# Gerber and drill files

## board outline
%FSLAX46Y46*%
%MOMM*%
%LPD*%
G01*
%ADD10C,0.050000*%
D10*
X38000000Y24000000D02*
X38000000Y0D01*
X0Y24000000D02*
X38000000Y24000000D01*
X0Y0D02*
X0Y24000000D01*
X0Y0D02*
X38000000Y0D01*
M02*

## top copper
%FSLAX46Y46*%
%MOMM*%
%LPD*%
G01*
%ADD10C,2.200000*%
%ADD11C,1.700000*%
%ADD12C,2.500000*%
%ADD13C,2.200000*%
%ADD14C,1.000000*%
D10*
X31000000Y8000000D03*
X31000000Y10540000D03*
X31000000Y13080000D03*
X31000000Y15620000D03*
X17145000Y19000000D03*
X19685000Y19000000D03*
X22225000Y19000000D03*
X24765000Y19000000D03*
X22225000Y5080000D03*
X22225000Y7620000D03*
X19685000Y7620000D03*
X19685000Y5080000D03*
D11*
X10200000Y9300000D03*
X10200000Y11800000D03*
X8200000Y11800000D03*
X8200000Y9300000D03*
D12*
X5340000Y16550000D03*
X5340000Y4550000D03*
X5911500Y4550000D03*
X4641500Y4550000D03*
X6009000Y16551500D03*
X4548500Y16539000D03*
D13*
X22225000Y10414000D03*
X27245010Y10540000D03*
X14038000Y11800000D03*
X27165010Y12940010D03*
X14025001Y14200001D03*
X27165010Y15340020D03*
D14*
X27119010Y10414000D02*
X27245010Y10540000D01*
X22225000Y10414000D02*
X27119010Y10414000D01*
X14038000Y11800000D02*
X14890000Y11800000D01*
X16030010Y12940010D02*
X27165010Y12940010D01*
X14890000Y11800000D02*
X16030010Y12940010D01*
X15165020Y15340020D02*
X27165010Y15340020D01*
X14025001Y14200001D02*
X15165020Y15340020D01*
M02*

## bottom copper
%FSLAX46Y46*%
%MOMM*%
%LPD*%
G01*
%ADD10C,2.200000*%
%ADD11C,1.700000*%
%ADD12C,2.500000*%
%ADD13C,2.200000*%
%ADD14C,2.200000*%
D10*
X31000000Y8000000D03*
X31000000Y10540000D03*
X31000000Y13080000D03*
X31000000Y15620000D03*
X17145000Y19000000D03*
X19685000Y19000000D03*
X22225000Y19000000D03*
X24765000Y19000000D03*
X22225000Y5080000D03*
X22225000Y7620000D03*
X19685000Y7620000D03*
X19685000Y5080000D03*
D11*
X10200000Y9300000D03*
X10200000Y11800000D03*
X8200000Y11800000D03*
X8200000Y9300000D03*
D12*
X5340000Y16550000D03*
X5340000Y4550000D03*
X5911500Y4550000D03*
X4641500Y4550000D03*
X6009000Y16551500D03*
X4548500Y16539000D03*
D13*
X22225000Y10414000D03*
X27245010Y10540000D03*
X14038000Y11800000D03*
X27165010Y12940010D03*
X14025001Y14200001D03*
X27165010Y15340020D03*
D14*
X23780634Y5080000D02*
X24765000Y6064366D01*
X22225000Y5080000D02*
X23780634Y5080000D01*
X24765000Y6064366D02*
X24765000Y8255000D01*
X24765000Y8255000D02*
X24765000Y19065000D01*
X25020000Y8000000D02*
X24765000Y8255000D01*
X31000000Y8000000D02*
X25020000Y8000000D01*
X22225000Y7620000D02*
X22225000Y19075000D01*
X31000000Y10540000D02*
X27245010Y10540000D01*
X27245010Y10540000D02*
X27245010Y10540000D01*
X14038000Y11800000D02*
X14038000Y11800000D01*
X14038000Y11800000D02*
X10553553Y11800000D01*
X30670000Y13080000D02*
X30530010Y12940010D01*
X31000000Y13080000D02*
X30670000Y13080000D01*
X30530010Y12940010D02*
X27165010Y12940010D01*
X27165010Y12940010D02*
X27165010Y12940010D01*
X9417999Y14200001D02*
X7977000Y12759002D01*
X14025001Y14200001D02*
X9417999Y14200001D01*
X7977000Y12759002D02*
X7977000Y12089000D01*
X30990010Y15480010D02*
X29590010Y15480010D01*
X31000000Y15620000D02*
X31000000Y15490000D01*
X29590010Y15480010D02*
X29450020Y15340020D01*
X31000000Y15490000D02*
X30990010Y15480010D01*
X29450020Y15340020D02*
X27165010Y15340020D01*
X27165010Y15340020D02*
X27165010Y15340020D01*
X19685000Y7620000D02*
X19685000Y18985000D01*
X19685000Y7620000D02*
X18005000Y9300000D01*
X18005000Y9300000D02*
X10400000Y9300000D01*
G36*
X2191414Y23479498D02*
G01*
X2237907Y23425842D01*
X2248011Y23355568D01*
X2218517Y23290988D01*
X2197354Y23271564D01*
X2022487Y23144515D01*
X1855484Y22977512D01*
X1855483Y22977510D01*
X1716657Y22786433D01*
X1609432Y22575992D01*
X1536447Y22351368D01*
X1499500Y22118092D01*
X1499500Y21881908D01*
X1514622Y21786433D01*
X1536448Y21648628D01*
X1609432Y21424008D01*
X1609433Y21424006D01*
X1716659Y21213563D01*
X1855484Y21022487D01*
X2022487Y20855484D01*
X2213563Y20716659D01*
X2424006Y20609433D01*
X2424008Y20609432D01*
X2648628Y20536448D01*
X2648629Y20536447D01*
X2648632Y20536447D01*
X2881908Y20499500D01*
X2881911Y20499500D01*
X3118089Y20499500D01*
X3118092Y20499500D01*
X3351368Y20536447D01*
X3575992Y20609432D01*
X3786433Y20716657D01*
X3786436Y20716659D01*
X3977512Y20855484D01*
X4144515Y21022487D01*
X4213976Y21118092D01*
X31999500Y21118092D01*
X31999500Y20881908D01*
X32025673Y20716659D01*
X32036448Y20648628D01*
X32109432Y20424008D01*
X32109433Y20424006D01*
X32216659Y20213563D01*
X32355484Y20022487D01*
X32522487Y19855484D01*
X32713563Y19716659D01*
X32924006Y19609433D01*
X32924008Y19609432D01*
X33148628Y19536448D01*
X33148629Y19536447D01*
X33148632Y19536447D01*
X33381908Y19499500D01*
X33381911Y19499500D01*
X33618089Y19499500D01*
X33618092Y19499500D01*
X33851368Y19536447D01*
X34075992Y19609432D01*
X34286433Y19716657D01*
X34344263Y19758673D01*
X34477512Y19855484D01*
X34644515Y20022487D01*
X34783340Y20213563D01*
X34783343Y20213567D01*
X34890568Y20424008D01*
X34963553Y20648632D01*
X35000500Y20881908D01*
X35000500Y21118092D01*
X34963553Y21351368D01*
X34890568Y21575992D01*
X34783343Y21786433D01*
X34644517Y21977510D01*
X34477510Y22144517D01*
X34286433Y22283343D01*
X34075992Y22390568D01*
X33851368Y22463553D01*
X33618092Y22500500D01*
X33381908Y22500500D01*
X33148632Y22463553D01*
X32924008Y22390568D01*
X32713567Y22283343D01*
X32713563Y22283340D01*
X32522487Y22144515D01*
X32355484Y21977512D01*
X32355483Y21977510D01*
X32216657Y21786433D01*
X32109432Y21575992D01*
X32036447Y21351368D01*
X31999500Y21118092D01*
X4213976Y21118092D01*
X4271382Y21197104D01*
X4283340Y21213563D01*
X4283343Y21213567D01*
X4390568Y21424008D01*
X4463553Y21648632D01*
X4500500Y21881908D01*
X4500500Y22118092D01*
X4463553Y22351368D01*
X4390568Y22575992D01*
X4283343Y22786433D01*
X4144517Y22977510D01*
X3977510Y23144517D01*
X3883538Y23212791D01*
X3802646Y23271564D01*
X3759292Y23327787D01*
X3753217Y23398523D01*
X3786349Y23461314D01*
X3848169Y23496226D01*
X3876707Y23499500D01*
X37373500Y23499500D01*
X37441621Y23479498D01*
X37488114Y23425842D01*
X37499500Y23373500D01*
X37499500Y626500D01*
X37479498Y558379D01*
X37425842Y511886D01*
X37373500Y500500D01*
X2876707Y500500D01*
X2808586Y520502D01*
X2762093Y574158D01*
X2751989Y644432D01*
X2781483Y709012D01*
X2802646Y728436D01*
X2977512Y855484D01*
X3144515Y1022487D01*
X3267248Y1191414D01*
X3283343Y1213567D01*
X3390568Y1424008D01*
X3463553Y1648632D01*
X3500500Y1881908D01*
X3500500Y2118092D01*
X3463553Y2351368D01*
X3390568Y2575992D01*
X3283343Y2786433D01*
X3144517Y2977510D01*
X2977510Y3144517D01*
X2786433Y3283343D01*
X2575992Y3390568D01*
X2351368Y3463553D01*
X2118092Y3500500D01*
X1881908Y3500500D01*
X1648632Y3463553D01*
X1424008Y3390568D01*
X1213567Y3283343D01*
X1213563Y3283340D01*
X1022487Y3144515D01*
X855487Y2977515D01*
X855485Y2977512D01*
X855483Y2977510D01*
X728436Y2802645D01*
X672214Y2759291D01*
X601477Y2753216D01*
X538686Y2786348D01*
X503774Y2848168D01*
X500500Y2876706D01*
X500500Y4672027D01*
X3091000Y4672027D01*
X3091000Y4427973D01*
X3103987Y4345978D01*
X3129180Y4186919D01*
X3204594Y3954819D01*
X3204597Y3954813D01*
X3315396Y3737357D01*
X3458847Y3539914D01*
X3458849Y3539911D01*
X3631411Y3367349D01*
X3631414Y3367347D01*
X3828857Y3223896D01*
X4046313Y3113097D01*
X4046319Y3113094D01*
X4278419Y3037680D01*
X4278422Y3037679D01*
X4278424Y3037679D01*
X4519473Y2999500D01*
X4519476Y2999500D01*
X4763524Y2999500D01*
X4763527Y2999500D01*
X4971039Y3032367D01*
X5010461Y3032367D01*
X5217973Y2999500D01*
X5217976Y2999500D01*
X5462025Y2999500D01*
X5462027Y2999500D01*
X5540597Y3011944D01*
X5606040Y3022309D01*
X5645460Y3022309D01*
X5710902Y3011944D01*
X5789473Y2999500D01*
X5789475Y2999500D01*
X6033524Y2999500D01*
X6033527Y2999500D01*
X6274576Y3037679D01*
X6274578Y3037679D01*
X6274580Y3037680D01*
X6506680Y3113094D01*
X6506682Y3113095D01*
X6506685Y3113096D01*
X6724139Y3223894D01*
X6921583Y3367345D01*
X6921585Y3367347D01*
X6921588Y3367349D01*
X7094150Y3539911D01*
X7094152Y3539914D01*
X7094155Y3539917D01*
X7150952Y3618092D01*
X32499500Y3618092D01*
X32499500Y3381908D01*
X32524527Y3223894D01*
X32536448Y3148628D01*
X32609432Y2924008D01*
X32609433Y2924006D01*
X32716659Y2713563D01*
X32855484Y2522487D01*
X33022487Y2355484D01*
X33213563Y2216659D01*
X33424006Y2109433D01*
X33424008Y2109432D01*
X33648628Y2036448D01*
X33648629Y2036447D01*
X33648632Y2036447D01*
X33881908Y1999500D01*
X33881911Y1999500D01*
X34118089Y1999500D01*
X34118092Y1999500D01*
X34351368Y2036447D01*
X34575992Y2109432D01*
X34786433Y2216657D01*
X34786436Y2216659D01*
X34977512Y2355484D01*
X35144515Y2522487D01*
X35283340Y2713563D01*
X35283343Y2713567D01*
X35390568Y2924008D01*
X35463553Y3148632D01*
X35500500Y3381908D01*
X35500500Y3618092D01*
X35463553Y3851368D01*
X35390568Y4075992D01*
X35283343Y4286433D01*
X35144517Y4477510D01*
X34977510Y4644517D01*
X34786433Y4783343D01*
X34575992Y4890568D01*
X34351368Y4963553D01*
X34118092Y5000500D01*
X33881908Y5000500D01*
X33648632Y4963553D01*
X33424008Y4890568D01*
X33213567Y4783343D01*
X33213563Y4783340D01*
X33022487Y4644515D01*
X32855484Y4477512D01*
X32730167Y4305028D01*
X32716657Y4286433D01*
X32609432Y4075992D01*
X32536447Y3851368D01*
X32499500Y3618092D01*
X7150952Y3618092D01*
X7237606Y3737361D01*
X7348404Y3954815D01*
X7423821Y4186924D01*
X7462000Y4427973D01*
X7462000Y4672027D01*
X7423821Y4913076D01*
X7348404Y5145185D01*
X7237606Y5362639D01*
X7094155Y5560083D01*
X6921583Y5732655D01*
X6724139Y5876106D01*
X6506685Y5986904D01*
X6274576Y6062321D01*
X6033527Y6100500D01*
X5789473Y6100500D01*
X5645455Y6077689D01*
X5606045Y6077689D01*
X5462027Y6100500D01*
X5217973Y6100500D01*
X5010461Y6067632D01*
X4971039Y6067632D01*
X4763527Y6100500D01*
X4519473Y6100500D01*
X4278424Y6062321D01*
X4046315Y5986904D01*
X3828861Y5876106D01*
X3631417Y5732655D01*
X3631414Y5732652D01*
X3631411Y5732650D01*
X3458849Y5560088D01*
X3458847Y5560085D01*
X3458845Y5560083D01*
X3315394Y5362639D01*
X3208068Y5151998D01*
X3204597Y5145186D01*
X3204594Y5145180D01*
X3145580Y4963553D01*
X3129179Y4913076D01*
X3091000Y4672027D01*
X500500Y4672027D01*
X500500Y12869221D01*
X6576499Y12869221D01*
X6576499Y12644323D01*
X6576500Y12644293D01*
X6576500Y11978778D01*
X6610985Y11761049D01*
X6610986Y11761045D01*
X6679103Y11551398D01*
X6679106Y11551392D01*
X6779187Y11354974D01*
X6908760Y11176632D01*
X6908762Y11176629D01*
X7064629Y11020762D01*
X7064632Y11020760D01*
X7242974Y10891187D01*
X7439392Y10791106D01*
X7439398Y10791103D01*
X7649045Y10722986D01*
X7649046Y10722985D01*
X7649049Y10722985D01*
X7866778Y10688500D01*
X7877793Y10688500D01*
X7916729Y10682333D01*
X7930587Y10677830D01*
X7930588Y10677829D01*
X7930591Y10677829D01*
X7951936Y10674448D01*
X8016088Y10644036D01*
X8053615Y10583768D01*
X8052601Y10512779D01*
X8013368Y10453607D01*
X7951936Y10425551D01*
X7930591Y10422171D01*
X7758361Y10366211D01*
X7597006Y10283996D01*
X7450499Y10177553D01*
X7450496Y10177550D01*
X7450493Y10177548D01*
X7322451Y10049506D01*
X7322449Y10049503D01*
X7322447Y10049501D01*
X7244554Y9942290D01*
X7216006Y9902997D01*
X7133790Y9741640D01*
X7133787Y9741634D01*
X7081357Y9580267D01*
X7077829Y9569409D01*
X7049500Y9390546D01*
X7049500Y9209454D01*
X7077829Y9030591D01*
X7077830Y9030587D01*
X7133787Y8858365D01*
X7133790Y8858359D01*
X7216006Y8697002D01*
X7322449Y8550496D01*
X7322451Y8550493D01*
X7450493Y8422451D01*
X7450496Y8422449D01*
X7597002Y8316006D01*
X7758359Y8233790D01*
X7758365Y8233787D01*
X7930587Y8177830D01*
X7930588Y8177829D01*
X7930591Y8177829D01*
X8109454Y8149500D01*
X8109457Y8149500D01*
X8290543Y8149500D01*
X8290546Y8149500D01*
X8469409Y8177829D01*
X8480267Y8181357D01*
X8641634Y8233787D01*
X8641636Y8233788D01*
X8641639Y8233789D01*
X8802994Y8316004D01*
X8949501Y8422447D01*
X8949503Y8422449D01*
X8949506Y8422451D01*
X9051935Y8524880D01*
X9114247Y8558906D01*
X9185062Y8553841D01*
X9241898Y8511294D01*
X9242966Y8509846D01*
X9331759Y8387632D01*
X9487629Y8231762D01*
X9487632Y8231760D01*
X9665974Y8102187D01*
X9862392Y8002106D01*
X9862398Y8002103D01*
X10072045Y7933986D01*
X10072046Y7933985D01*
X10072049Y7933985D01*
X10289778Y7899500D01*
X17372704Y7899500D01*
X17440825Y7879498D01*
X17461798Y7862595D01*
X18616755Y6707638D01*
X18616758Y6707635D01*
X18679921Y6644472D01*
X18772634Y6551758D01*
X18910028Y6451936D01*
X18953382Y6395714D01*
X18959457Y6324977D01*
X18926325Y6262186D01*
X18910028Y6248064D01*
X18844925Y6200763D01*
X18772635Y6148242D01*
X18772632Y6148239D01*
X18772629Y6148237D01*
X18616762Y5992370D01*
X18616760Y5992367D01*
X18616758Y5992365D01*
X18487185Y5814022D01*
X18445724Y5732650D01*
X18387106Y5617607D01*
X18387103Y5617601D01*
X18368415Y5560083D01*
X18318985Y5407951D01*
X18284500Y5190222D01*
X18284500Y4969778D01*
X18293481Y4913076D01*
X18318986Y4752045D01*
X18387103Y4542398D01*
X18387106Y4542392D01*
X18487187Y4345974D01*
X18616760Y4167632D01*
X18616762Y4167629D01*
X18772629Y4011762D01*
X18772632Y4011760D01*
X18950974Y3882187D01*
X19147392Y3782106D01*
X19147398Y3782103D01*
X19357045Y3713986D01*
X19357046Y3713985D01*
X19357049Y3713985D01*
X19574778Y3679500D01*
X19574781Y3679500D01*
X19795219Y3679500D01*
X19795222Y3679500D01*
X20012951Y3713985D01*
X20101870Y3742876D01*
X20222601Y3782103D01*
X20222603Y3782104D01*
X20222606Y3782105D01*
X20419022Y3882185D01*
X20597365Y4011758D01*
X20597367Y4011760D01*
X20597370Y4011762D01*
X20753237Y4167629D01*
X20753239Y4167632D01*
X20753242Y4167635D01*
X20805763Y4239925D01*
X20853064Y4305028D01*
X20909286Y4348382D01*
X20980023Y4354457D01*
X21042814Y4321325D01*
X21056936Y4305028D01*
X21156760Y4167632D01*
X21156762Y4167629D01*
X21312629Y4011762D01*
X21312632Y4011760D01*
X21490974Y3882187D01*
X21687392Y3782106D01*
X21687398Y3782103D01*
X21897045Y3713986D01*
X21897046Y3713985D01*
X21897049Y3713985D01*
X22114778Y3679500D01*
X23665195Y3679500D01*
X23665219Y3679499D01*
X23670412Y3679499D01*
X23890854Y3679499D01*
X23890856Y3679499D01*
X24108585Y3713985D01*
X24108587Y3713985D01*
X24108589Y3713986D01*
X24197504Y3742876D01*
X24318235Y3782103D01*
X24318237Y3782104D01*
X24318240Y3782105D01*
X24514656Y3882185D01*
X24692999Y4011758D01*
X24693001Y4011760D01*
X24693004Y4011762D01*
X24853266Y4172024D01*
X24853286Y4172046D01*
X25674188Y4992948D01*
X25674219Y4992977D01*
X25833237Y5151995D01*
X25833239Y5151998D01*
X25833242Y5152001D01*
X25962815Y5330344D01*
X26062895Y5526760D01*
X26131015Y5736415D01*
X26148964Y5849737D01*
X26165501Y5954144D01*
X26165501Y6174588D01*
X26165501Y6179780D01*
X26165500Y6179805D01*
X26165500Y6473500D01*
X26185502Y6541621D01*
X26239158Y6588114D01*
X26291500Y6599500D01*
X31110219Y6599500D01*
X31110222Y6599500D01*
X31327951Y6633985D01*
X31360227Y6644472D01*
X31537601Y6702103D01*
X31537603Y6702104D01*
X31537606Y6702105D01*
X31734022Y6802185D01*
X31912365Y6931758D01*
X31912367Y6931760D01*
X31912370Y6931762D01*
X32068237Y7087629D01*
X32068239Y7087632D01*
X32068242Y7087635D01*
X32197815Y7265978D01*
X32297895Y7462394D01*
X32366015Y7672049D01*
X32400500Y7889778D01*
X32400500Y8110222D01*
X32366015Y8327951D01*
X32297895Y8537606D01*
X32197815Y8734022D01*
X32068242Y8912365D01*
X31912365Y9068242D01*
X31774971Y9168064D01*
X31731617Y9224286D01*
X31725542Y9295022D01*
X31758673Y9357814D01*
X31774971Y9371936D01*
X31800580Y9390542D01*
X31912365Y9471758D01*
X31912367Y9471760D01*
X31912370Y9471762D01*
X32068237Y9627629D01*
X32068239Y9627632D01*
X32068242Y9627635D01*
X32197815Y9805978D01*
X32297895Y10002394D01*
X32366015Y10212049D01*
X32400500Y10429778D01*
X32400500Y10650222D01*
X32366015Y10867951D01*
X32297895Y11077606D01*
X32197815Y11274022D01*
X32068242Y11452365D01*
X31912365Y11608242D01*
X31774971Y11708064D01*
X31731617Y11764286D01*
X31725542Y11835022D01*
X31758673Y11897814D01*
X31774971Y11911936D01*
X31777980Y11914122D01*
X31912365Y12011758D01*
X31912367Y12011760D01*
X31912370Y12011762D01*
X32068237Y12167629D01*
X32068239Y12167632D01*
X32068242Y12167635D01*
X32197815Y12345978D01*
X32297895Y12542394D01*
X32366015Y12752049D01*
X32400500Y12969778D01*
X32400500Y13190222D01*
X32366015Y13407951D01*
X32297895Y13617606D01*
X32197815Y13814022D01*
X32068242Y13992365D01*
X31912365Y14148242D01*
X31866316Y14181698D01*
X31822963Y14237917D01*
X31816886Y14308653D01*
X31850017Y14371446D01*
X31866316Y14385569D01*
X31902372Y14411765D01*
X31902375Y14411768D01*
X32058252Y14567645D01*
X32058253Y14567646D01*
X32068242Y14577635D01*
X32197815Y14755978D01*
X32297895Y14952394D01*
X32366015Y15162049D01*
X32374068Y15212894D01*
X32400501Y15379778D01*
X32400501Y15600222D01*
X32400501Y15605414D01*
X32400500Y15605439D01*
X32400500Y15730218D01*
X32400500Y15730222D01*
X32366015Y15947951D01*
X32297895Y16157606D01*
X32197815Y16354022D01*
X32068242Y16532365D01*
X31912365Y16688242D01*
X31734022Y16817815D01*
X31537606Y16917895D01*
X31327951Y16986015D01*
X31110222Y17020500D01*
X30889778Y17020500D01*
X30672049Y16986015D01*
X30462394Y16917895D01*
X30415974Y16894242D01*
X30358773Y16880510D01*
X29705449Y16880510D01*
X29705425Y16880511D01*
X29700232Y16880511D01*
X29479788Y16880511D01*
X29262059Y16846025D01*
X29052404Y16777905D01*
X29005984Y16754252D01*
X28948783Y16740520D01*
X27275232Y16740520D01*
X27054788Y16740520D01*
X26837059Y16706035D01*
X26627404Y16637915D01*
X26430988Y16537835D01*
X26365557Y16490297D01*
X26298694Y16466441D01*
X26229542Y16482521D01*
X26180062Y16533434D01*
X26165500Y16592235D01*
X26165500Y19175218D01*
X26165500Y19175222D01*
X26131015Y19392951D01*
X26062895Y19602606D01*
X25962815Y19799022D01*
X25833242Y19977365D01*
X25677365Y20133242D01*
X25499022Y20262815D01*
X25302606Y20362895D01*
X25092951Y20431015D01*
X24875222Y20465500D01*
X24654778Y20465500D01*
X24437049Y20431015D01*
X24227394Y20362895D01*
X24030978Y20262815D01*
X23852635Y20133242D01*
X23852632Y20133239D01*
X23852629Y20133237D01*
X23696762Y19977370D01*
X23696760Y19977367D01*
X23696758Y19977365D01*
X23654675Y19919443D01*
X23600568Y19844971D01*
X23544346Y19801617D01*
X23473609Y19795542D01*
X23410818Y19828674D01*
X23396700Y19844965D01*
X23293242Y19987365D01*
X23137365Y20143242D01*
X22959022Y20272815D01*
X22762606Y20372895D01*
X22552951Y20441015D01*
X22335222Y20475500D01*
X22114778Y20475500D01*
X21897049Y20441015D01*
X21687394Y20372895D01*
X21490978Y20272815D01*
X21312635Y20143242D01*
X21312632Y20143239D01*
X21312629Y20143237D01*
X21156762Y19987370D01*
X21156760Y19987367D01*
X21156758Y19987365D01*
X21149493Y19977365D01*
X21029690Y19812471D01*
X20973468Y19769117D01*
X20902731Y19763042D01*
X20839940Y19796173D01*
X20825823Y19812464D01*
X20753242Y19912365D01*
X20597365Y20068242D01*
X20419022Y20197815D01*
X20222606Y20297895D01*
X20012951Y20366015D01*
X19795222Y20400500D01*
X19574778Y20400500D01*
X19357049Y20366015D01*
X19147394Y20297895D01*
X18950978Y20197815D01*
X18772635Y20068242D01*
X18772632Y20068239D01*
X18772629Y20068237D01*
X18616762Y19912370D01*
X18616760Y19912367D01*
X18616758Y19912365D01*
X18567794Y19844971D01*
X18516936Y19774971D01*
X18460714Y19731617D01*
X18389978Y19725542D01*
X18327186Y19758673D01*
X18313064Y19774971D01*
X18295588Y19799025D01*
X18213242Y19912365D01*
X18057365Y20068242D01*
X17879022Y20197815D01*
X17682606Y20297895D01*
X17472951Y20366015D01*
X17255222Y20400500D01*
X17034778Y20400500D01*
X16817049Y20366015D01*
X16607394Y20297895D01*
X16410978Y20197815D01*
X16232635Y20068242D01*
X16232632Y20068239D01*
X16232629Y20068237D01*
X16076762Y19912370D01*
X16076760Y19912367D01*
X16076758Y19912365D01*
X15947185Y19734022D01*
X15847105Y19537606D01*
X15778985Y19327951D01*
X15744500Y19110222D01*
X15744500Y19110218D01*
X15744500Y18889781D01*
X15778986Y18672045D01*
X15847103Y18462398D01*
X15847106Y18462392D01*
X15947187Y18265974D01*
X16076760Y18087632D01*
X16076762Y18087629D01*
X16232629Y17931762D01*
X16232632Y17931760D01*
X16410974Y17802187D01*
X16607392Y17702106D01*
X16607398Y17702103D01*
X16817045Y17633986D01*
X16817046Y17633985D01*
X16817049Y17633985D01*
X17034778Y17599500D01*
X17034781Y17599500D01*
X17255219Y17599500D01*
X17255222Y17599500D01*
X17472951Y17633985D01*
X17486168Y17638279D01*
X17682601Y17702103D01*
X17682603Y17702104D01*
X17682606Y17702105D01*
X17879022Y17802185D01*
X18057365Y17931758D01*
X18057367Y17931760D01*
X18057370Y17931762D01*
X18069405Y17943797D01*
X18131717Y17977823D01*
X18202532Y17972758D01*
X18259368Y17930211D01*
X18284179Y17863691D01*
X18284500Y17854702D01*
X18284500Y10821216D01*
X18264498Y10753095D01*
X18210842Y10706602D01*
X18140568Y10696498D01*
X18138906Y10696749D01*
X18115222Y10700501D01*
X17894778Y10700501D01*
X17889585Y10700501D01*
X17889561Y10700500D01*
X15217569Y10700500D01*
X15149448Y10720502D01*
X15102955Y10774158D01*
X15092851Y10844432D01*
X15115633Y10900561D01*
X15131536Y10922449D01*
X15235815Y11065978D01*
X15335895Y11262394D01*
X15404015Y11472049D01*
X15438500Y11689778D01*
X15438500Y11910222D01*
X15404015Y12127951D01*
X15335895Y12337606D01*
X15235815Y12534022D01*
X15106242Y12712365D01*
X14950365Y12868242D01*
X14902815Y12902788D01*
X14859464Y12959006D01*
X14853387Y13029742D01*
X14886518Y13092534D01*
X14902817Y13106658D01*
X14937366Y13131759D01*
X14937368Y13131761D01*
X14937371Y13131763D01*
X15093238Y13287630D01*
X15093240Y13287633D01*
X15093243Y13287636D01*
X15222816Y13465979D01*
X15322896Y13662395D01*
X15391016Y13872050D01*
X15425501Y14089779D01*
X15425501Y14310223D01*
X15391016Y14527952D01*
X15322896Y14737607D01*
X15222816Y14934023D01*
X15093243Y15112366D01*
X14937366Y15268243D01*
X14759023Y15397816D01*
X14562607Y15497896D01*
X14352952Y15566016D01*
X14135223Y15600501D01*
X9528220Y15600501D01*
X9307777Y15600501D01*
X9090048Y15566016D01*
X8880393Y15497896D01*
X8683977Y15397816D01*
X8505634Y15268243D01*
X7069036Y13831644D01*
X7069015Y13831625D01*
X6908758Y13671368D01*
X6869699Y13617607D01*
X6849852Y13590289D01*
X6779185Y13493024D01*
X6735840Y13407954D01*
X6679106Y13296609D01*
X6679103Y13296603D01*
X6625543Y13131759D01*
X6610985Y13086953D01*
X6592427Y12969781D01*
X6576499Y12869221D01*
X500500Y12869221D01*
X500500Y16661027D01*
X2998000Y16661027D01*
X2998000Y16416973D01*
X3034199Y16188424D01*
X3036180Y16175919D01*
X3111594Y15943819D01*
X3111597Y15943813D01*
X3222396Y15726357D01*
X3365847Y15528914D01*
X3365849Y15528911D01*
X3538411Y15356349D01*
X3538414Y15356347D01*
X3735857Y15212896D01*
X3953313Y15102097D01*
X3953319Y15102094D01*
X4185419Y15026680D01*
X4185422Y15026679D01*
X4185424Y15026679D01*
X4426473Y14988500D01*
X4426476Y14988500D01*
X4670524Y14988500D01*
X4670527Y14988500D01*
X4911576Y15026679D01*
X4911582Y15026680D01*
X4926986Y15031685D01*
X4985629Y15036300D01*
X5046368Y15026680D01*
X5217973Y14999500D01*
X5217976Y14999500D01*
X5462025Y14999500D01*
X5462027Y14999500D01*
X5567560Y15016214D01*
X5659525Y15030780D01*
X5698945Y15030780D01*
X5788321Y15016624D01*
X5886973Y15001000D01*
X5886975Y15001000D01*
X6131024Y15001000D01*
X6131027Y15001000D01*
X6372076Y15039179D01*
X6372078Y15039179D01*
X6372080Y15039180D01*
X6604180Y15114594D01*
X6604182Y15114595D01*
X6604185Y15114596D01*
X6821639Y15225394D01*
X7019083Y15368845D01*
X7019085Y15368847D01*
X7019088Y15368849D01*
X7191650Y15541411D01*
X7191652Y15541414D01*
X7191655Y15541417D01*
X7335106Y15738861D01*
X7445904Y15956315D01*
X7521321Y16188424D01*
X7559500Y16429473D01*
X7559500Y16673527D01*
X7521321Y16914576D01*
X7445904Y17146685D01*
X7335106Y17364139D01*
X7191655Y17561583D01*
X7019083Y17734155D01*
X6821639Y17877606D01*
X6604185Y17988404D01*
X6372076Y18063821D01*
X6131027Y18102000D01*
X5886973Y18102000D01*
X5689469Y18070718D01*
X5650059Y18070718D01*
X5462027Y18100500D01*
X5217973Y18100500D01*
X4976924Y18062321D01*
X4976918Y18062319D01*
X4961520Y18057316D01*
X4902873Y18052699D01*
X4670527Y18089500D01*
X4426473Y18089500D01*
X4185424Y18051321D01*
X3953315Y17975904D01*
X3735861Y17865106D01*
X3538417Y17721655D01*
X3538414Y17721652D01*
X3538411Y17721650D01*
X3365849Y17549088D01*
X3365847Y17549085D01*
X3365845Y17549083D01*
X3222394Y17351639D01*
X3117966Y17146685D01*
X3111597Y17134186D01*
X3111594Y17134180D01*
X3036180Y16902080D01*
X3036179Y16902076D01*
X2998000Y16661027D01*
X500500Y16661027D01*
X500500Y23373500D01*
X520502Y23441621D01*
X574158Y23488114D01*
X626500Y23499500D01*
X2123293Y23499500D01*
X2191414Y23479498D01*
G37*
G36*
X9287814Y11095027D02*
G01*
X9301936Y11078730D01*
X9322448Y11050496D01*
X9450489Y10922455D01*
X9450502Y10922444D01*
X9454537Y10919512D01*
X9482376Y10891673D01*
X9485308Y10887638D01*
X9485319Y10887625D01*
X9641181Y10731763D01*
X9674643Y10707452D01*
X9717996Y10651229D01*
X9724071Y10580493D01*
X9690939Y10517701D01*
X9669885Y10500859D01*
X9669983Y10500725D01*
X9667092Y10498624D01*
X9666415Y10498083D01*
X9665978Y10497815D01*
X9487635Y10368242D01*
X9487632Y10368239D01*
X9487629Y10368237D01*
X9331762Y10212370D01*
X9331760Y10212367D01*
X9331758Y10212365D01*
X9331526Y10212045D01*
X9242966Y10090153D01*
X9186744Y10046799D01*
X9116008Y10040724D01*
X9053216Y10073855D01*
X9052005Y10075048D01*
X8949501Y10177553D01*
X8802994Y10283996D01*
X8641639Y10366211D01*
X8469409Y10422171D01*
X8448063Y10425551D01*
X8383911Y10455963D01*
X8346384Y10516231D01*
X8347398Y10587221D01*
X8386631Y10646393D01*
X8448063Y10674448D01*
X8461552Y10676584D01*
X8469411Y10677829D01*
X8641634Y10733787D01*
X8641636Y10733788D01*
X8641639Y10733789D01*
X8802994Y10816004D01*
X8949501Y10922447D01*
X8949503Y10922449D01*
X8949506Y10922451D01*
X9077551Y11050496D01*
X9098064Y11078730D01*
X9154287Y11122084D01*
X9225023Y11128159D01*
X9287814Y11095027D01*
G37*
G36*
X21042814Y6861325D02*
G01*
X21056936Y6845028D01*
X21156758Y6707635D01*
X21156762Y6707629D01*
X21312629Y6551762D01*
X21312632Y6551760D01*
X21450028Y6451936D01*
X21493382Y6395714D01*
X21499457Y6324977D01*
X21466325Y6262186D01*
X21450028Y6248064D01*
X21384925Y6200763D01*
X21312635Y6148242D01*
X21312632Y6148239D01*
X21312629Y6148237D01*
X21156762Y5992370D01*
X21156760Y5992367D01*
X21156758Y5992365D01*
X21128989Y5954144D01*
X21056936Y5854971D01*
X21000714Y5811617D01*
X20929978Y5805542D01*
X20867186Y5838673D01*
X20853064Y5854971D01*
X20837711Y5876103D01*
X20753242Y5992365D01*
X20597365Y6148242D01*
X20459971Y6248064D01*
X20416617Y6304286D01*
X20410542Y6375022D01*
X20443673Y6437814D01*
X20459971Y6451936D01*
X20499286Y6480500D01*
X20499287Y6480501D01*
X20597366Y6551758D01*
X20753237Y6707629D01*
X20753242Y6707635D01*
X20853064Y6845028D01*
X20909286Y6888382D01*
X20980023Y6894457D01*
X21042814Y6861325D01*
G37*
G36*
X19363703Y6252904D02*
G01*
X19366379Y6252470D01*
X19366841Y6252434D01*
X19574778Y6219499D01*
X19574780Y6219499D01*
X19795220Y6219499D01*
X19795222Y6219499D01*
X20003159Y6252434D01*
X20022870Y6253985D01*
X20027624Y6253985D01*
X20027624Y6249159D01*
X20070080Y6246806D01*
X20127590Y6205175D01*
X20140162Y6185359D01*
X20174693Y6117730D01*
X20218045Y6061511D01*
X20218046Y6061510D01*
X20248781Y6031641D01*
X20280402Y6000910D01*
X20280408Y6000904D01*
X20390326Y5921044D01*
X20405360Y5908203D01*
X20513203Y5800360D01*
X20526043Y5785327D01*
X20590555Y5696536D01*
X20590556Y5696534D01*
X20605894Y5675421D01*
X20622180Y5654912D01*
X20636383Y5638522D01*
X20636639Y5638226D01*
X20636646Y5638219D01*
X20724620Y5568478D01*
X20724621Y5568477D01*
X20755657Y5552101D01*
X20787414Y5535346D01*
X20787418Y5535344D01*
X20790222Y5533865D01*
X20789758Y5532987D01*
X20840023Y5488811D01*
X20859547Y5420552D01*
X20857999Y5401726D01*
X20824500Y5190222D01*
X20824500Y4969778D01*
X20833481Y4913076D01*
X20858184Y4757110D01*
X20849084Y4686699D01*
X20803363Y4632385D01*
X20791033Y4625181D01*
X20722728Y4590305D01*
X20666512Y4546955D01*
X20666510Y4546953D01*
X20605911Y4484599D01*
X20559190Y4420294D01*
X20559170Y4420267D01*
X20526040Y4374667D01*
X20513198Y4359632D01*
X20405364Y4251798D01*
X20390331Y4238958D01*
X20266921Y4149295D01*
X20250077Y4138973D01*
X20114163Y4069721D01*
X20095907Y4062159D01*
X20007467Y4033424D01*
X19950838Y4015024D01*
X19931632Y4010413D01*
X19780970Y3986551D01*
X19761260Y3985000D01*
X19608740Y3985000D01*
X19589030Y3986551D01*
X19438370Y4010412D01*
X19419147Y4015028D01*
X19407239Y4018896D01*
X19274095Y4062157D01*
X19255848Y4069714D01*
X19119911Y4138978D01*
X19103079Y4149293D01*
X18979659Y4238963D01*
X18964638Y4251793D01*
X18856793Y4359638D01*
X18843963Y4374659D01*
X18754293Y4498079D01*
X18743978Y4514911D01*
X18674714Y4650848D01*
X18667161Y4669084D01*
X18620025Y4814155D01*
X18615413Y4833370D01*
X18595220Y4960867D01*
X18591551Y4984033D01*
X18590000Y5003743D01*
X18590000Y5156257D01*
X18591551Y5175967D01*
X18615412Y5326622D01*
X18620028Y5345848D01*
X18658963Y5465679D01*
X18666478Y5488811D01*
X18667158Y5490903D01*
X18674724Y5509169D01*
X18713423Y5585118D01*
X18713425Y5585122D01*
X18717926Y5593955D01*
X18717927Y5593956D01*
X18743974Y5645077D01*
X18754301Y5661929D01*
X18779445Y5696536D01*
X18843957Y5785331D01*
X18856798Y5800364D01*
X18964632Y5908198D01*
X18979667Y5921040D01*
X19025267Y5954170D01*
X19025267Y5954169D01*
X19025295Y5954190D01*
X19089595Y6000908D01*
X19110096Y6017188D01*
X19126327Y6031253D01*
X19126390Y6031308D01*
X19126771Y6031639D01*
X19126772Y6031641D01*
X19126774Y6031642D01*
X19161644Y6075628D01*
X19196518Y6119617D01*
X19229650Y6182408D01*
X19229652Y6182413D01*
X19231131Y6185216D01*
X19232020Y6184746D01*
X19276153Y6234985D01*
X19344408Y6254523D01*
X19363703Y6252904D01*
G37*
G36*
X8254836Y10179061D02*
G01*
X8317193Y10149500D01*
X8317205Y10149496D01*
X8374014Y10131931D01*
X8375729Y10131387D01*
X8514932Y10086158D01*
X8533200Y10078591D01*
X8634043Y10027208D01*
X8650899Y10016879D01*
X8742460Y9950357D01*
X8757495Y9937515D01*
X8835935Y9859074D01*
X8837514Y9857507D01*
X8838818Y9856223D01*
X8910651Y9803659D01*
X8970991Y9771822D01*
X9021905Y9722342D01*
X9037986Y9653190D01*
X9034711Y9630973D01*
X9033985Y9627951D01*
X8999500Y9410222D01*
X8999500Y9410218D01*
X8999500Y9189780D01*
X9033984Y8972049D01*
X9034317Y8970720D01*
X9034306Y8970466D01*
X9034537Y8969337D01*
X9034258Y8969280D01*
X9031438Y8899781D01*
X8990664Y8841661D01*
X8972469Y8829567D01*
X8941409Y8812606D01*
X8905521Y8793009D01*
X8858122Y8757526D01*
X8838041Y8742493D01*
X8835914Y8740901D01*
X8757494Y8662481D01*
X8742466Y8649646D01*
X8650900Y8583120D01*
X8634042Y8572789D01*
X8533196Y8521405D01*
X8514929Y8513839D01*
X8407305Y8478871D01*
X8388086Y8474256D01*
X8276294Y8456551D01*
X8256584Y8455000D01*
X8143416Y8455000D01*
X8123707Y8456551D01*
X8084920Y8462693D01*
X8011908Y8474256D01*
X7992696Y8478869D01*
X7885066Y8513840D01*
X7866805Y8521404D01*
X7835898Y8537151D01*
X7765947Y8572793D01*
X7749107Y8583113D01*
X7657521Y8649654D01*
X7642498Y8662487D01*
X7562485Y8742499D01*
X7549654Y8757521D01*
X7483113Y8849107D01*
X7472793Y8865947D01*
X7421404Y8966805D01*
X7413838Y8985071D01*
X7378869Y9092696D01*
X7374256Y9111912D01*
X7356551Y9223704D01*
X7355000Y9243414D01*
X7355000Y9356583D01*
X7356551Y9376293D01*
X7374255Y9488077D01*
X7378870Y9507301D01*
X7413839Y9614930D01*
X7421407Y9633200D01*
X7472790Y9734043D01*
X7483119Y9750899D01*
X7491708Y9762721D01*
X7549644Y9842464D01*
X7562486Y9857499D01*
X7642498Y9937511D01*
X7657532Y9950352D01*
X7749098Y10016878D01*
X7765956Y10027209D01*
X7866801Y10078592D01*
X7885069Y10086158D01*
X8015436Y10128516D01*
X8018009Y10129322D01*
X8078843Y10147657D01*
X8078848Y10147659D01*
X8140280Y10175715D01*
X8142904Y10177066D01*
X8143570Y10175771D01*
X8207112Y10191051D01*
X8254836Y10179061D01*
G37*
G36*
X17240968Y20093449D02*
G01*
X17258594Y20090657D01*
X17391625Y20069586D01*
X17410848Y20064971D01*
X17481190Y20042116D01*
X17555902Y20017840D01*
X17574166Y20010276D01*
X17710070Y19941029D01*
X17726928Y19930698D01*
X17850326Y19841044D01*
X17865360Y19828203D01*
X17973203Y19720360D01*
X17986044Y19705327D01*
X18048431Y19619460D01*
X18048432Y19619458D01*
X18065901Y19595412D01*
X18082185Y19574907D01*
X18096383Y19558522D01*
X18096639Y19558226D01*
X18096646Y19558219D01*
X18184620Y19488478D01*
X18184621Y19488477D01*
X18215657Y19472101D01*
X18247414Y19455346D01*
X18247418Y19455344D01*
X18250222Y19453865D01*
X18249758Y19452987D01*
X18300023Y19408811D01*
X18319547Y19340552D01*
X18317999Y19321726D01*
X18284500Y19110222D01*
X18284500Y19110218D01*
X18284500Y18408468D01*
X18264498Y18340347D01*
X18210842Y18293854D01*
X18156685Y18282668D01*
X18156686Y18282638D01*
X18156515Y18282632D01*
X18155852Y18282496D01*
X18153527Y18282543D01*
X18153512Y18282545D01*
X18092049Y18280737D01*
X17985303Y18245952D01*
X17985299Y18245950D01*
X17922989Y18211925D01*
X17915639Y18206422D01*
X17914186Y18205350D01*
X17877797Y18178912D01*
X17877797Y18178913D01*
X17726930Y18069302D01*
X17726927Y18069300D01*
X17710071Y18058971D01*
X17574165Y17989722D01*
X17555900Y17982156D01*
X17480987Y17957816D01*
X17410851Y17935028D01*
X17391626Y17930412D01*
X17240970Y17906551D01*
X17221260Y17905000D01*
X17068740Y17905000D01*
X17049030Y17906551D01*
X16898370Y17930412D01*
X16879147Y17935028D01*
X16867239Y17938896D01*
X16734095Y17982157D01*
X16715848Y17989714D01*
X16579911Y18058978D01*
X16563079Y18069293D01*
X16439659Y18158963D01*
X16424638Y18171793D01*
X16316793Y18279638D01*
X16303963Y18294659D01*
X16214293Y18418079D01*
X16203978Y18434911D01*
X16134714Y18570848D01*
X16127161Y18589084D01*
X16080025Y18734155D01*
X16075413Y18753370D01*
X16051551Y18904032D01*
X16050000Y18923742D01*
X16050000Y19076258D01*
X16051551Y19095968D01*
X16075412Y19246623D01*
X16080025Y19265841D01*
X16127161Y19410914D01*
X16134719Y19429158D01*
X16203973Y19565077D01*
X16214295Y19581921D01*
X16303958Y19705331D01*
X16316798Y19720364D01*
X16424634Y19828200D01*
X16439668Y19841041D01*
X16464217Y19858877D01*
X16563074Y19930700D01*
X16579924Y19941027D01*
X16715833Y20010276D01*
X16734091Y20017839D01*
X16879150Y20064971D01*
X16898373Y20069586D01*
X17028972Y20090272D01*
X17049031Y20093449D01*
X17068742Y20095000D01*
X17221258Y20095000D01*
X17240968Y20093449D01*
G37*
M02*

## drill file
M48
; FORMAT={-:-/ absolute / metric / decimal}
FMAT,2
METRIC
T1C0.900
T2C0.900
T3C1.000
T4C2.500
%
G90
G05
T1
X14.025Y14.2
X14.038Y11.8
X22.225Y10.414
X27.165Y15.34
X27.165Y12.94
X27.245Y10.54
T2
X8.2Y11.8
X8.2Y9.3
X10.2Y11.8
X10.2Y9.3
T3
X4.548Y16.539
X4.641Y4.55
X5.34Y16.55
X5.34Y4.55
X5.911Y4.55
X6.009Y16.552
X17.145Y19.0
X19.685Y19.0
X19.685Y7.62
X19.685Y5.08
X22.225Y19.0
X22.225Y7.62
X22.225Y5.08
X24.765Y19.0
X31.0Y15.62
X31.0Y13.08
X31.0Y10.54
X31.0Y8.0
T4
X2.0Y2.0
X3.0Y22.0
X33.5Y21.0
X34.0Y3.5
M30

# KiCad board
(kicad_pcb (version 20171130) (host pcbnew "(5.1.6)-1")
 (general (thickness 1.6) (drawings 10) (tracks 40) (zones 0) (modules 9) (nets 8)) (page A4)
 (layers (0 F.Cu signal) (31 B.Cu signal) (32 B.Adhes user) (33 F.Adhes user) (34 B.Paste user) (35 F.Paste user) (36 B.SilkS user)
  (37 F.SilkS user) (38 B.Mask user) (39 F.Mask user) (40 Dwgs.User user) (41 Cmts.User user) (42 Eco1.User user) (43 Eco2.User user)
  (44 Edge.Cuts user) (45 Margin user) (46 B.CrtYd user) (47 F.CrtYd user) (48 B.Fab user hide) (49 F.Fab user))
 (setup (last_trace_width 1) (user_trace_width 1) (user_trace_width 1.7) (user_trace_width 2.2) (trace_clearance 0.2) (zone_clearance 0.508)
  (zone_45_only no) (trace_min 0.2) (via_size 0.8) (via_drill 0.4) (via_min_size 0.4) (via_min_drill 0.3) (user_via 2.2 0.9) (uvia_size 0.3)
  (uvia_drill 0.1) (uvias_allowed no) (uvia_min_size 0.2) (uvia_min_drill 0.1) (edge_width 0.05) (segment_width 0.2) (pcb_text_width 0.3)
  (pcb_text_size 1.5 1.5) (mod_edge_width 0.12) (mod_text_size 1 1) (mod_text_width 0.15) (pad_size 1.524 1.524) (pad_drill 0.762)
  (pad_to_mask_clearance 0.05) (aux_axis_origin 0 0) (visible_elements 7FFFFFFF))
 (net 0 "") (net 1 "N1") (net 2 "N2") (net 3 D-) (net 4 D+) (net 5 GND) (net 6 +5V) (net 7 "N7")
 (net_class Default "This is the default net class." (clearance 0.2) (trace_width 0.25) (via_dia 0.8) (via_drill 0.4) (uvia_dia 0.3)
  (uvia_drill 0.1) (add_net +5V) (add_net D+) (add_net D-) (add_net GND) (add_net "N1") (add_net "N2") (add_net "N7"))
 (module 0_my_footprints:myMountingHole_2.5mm (layer F.Cu) (at 3 -22)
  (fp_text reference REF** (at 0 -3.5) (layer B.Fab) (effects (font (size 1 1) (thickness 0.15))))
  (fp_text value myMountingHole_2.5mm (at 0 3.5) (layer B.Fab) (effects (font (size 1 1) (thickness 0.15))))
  (pad 1 np_thru_hole circle (at 0 0) (size 2.5 2.5) (drill 2.5) (layers *.Cu *.Mask)))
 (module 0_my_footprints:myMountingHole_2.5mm (layer F.Cu) (at 33.5 -21)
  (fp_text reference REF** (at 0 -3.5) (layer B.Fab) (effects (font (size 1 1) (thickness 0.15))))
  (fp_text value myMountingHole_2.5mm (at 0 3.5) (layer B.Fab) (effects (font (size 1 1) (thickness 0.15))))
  (pad 1 np_thru_hole circle (at 0 0) (size 2.5 2.5) (drill 2.5) (layers *.Cu *.Mask)))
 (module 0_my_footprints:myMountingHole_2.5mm (layer F.Cu) (at 34 -3.5)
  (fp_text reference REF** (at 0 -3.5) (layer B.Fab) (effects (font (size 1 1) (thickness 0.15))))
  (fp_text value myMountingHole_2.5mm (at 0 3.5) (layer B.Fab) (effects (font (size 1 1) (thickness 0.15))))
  (pad 1 np_thru_hole circle (at 0 0) (size 2.5 2.5) (drill 2.5) (layers *.Cu *.Mask)))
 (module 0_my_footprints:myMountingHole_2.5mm (layer F.Cu) (at 2 -2)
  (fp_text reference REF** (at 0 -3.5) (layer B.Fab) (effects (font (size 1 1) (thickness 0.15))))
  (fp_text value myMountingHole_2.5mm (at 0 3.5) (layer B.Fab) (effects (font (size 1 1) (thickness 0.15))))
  (pad 1 np_thru_hole circle (at 0 0) (size 2.5 2.5) (drill 2.5) (layers *.Cu *.Mask)))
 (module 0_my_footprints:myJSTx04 (layer F.Cu) (at 31 -8 90)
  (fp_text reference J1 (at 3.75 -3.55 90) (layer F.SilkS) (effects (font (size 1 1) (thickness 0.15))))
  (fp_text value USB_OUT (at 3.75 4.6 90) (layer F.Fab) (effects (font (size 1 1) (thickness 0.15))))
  (pad 1 thru_hole circle (at 0 0 90) (size 2.2 2.2) (drill 1) (layers *.Cu *.Mask) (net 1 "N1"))
  (pad 2 thru_hole circle (at 2.54 0 90) (size 2.2 2.2) (drill 1) (layers *.Cu *.Mask) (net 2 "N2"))
  (pad 3 thru_hole circle (at 5.08 0 90) (size 2.2 2.2) (drill 1) (layers *.Cu *.Mask) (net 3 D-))
  (pad 4 thru_hole circle (at 7.62 0 90) (size 2.2 2.2) (drill 1) (layers *.Cu *.Mask) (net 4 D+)))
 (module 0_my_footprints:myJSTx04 (layer F.Cu) (at 24.765 -19 180)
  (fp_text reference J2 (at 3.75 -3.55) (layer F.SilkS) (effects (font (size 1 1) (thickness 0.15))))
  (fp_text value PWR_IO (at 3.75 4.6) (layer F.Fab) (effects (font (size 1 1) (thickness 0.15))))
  (pad 4 thru_hole circle (at 7.62 0 180) (size 2.2 2.2) (drill 1) (layers *.Cu *.Mask) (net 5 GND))
  (pad 3 thru_hole circle (at 5.08 0 180) (size 2.2 2.2) (drill 1) (layers *.Cu *.Mask) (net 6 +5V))
  (pad 2 thru_hole circle (at 2.54 0 180) (size 2.2 2.2) (drill 1) (layers *.Cu *.Mask) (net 2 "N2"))
  (pad 1 thru_hole circle (at 0 0 180) (size 2.2 2.2) (drill 1) (layers *.Cu *.Mask) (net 1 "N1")))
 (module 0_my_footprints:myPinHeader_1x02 (layer F.Cu) (at 22.225 -5.08 180)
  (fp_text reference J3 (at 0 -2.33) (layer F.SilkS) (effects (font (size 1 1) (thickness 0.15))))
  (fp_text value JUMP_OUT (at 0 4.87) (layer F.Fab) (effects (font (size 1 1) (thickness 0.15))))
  (pad 1 thru_hole circle (at 0 0 180) (size 2.2 2.2) (drill 1) (layers *.Cu *.Mask) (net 1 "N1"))
  (pad 2 thru_hole circle (at 0 2.54 180) (size 2.2 2.2) (drill 1) (layers *.Cu *.Mask) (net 2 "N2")))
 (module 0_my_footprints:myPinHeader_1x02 (layer F.Cu) (at 19.685 -5.08 180)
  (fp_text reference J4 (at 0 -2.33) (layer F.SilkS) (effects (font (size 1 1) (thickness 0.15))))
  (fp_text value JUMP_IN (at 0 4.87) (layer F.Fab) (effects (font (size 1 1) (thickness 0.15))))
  (pad 2 thru_hole circle (at 0 2.54 180) (size 2.2 2.2) (drill 1) (layers *.Cu *.Mask) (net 6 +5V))
  (pad 1 thru_hole circle (at 0 0 180) (size 2.2 2.2) (drill 1) (layers *.Cu *.Mask) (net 5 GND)))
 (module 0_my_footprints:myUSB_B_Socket (layer F.Cu) (at 10.2 -9.3 180)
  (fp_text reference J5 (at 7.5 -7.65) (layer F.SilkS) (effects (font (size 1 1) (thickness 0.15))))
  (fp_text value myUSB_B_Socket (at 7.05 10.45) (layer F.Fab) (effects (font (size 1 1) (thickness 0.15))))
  (pad 1 thru_hole circle (at 0 0 270) (size 1.7 1.7) (drill 0.9) (layers *.Cu *.Mask) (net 6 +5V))
  (pad 2 thru_hole circle (at 0 2.5 270) (size 1.7 1.7) (drill 0.9) (layers *.Cu *.Mask) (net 3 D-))
  (pad 3 thru_hole circle (at 2 2.5 270) (size 1.7 1.7) (drill 0.9) (layers *.Cu *.Mask) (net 4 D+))
  (pad 4 thru_hole circle (at 2 0 270) (size 1.7 1.7) (drill 0.9) (layers *.Cu *.Mask) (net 5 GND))
  (pad 5 thru_hole circle (at 4.86 7.25 270) (size 2.5 2.5) (drill 1) (layers *.Cu *.Mask) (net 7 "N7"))
  (pad 5 thru_hole circle (at 4.86 -4.75 270) (size 2.5 2.5) (drill 1) (layers *.Cu *.Mask) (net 7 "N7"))
  (pad 5 thru_hole circle (at 4.2885 -4.75 270) (size 2.5 2.5) (drill 1) (layers *.Cu *.Mask) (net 7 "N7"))
  (pad 5 thru_hole circle (at 5.5585 -4.75 270) (size 2.5 2.5) (drill 1) (layers *.Cu *.Mask) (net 7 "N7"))
  (pad 5 thru_hole circle (at 4.191 7.2515 270) (size 2.5 2.5) (drill 1) (layers *.Cu *.Mask) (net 7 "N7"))
  (pad 5 thru_hole circle (at 5.6515 7.239 270) (size 2.5 2.5) (drill 1) (layers *.Cu *.Mask) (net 7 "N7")))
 (gr_line (start 38 -24) (end 38 0) (layer Edge.Cuts) (width 0.05))
 (gr_line (start 0 -24) (end 38 -24) (layer Edge.Cuts) (width 0.05))
 (gr_line (start 0 0) (end 0 -24) (layer Edge.Cuts) (width 0.05))
 (gr_line (start 0 0) (end 38 0) (layer Edge.Cuts) (width 0.05))
 (segment (start 23.780634 -5.08) (end 24.765 -6.064366) (width 2.2) (layer B.Cu) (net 1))
 (segment (start 22.225 -5.08) (end 23.780634 -5.08) (width 2.2) (layer B.Cu) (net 1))
 (segment (start 24.765 -6.064366) (end 24.765 -8.255) (width 2.2) (layer B.Cu) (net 1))
 (segment (start 24.765 -8.255) (end 24.765 -19.065) (width 2.2) (layer B.Cu) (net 1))
 (segment (start 25.02 -8) (end 24.765 -8.255) (width 2.2) (layer B.Cu) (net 1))
 (segment (start 31 -8) (end 25.02 -8) (width 2.2) (layer B.Cu) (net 1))
 (via (at 22.225 -10.414) (size 2.2) (drill 0.9) (layers F.Cu B.Cu) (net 2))
 (segment (start 22.225 -7.62) (end 22.225 -19.075) (width 2.2) (layer B.Cu) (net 2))
 (segment (start 31 -10.54) (end 27.24501 -10.54) (width 2.2) (layer B.Cu) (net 2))
 (segment (start 27.24501 -10.54) (end 27.24501 -10.54) (width 2.2) (layer B.Cu) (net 2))
 (via (at 27.24501 -10.54) (size 2.2) (drill 0.9) (layers F.Cu B.Cu) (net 2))
 (segment (start 27.11901 -10.414) (end 27.24501 -10.54) (width 1) (layer F.Cu) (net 2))
 (segment (start 22.225 -10.414) (end 27.11901 -10.414) (width 1) (layer F.Cu) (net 2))
 (segment (start 14.038 -11.8) (end 14.038 -11.8) (width 2.2) (layer B.Cu) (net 3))
 (segment (start 14.038 -11.8) (end 10.553553 -11.8) (width 2.2) (layer B.Cu) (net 3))
 (via (at 14.038 -11.8) (size 2.2) (drill 0.9) (layers F.Cu B.Cu) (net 3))
 (segment (start 30.67 -13.08) (end 30.53001 -12.94001) (width 2.2) (layer B.Cu) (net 3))
 (segment (start 31 -13.08) (end 30.67 -13.08) (width 2.2) (layer B.Cu) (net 3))
 (segment (start 30.53001 -12.94001) (end 27.16501 -12.94001) (width 2.2) (layer B.Cu) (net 3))
 (segment (start 27.16501 -12.94001) (end 27.16501 -12.94001) (width 2.2) (layer B.Cu) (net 3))
 (via (at 27.16501 -12.94001) (size 2.2) (drill 0.9) (layers F.Cu B.Cu) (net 3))
 (segment (start 14.038 -11.8) (end 14.89 -11.8) (width 1) (layer F.Cu) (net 3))
 (segment (start 16.03001 -12.94001) (end 27.16501 -12.94001) (width 1) (layer F.Cu) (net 3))
 (segment (start 14.89 -11.8) (end 16.03001 -12.94001) (width 1) (layer F.Cu) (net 3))
 (via (at 14.025001 -14.200001) (size 2.2) (drill 0.9) (layers F.Cu B.Cu) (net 4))
 (segment (start 9.417999 -14.200001) (end 7.977 -12.759002) (width 2.2) (layer B.Cu) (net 4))
 (segment (start 14.025001 -14.200001) (end 9.417999 -14.200001) (width 2.2) (layer B.Cu) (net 4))
 (segment (start 7.977 -12.759002) (end 7.977 -12.089) (width 2.2) (layer B.Cu) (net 4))
 (segment (start 30.99001 -15.48001) (end 29.59001 -15.48001) (width 2.2) (layer B.Cu) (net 4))
 (segment (start 31 -15.62) (end 31 -15.49) (width 2.2) (layer B.Cu) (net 4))
 (segment (start 29.59001 -15.48001) (end 29.45002 -15.34002) (width 2.2) (layer B.Cu) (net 4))
 (segment (start 31 -15.49) (end 30.99001 -15.48001) (width 2.2) (layer B.Cu) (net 4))
 (segment (start 29.45002 -15.34002) (end 27.16501 -15.34002) (width 2.2) (layer B.Cu) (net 4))
 (segment (start 27.16501 -15.34002) (end 27.16501 -15.34002) (width 2.2) (layer B.Cu) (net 4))
 (via (at 27.16501 -15.34002) (size 2.2) (drill 0.9) (layers F.Cu B.Cu) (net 4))
 (segment (start 15.16502 -15.34002) (end 27.16501 -15.34002) (width 1) (layer F.Cu) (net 4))
 (segment (start 14.025001 -14.200001) (end 15.16502 -15.34002) (width 1) (layer F.Cu) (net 4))
 (segment (start 19.685 -7.62) (end 19.685 -18.985) (width 2.2) (layer B.Cu) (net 6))
 (segment (start 19.685 -7.62) (end 18.005 -9.3) (width 2.2) (layer B.Cu) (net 6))
 (segment (start 18.005 -9.3) (end 10.4 -9.3) (width 2.2) (layer B.Cu) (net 6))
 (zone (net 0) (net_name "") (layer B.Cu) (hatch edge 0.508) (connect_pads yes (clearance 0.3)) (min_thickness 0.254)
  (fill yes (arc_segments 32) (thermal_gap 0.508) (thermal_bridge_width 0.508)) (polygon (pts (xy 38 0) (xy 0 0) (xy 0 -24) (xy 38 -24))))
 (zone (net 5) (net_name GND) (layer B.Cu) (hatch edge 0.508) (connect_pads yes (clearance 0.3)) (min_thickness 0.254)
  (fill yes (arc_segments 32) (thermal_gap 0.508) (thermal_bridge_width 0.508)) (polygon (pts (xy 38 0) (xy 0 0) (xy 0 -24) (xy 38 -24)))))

